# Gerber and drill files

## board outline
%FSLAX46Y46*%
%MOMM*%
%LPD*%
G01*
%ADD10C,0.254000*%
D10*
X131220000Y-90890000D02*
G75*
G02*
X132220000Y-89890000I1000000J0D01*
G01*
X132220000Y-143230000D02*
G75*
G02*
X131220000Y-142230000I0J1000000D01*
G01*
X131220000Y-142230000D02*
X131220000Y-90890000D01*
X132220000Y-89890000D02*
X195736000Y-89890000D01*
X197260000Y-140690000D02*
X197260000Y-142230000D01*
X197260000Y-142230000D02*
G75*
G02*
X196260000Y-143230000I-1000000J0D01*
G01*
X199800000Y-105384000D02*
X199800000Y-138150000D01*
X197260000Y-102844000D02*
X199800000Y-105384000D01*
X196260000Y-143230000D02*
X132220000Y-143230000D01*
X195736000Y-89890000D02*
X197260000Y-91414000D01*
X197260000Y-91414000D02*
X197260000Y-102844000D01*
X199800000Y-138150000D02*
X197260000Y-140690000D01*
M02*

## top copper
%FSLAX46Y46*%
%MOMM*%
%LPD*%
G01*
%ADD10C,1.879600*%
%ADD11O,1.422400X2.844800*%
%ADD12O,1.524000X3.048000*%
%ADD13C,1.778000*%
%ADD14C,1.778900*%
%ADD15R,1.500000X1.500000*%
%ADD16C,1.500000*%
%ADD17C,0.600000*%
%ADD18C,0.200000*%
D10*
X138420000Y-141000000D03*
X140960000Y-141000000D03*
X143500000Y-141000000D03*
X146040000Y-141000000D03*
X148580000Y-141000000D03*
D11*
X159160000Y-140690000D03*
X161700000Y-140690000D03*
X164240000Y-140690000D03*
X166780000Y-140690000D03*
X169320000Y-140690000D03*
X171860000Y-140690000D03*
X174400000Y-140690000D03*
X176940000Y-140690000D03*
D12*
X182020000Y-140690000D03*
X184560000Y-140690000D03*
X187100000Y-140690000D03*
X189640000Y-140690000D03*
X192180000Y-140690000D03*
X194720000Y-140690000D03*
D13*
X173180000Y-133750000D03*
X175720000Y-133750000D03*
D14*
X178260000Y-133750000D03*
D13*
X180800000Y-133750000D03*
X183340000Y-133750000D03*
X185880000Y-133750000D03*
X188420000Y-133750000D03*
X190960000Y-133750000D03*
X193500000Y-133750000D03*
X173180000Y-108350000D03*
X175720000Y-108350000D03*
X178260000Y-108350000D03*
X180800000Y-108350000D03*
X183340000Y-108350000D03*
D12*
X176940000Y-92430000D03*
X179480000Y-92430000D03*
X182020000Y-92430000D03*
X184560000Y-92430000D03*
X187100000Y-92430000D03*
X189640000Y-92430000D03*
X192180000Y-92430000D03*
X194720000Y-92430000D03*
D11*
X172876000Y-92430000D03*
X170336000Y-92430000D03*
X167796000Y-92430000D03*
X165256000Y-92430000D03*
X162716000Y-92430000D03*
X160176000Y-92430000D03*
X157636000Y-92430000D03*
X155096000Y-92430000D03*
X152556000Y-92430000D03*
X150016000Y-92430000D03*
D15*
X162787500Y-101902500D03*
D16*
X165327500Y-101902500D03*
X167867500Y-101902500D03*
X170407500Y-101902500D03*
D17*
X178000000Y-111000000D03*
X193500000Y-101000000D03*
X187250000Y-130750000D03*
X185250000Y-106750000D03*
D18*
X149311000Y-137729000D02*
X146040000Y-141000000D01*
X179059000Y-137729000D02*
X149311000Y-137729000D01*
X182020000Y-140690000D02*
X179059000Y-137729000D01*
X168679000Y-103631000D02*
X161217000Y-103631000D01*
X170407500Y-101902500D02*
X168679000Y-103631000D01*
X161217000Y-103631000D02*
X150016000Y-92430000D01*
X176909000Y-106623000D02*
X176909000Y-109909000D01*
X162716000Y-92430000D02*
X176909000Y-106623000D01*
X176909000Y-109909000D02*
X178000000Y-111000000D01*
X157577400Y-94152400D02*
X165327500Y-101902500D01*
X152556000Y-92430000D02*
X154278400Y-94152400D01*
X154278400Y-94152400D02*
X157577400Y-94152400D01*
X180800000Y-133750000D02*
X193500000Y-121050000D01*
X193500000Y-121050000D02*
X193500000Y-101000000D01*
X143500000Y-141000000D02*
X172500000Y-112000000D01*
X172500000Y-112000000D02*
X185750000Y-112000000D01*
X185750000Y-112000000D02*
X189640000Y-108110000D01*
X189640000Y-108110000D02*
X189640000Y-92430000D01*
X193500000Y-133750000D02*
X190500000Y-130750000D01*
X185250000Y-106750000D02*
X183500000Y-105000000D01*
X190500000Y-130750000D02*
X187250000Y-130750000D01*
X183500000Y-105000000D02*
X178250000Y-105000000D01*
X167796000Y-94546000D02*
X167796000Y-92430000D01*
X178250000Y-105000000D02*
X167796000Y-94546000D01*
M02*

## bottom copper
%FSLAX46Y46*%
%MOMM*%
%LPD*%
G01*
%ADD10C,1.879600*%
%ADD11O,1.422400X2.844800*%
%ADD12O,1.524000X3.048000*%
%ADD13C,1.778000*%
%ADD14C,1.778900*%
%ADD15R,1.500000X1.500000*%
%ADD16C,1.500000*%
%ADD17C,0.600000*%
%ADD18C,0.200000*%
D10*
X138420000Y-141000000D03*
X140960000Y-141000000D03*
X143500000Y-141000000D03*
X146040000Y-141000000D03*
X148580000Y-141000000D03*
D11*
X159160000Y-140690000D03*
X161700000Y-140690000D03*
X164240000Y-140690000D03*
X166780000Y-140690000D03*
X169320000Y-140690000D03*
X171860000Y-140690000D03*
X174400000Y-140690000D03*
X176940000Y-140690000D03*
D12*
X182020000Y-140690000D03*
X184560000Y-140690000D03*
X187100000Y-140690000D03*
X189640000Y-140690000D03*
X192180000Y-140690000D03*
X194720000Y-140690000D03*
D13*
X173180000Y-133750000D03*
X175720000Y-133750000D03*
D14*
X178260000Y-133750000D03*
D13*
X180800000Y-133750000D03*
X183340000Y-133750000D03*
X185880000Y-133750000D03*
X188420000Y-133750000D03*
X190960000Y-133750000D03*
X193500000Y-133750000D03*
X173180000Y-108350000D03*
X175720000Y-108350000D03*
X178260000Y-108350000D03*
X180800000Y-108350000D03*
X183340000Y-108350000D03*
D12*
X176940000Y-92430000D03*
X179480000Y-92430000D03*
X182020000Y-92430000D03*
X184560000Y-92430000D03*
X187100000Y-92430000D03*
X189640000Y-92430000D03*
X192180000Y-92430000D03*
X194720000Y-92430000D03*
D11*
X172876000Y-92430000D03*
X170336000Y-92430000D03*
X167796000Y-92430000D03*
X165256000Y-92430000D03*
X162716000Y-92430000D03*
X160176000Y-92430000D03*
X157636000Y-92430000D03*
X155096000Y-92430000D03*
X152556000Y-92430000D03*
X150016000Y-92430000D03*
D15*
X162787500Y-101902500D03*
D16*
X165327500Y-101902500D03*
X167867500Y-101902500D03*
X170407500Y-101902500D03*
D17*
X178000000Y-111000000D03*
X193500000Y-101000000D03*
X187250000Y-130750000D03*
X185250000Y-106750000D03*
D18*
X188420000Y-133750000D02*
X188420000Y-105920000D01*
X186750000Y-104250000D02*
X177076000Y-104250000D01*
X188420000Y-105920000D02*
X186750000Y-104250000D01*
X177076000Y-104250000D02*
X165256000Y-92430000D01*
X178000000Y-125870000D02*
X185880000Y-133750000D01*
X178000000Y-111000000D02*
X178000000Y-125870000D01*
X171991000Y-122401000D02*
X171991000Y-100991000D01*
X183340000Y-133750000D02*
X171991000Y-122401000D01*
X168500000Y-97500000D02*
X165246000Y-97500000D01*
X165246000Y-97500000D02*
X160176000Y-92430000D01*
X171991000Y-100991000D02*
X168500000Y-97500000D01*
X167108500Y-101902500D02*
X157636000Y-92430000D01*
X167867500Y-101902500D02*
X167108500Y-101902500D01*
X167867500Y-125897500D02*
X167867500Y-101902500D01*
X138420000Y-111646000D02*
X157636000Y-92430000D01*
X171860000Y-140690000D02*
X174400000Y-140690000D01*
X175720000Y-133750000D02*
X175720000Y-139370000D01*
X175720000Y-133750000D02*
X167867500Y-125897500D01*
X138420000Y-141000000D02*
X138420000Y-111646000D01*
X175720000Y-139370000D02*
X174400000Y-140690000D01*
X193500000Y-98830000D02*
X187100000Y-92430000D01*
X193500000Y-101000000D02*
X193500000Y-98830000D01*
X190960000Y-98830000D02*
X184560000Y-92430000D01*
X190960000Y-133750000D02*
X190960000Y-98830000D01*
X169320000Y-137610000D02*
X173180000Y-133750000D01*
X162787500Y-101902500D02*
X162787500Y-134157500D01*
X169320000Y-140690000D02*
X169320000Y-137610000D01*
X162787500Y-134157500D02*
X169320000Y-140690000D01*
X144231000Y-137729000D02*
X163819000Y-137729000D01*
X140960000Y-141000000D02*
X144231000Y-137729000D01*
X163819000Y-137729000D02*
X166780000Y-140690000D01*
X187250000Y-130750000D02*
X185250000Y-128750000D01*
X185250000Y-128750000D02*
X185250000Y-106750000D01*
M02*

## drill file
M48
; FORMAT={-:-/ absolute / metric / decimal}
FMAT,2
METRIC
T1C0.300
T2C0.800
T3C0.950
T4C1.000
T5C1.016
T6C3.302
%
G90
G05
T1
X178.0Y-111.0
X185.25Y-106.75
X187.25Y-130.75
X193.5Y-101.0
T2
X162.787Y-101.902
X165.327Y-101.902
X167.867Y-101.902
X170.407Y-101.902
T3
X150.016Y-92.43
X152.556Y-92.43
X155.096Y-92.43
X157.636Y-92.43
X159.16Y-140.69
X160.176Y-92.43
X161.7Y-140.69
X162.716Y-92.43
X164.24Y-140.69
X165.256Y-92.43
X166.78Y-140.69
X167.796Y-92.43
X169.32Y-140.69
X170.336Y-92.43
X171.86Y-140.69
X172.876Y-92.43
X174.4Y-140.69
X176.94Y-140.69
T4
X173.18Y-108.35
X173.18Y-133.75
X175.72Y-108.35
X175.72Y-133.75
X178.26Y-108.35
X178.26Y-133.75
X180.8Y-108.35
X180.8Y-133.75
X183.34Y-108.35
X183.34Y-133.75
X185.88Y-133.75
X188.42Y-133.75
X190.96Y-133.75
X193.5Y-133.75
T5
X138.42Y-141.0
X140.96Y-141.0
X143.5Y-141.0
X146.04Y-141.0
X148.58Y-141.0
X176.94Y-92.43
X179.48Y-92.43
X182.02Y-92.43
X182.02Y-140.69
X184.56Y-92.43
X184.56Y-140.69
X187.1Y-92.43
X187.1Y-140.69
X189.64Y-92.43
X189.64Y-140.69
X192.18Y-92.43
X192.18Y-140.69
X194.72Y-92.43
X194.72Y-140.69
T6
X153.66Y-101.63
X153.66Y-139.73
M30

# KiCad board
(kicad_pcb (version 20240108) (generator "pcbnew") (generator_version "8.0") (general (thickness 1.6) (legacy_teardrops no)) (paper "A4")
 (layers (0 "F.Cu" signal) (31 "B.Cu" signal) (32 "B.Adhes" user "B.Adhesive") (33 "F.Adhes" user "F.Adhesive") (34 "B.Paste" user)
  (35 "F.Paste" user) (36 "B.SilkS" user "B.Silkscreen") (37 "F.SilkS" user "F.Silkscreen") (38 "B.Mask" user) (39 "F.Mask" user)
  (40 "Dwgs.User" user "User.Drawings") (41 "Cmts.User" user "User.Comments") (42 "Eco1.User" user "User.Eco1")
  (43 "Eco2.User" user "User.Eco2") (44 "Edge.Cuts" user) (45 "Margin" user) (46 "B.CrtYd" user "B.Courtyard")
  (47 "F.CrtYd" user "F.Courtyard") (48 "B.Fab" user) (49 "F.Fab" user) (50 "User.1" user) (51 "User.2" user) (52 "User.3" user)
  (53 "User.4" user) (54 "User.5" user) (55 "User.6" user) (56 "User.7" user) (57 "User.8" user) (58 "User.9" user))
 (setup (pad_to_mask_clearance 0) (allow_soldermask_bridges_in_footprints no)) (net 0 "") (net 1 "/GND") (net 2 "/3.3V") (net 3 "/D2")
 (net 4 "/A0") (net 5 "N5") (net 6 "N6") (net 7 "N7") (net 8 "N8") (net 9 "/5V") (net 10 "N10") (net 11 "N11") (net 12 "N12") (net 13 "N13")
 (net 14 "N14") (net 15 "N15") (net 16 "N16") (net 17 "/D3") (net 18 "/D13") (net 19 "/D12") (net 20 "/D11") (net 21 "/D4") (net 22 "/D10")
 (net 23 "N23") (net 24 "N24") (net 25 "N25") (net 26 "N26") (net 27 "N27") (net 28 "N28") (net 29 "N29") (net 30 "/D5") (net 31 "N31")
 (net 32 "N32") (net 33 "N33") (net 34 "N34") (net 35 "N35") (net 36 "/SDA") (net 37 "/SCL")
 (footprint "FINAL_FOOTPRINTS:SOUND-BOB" (layer "F.Cu") (at 249.7736 -27.8211 -90)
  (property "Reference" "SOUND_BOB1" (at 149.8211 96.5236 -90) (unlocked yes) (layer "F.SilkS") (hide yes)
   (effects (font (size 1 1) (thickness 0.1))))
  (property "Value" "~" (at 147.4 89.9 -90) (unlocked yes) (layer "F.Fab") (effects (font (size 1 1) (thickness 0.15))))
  (pad "" np_thru_hole circle (at 129.4511 96.1136 270) (size 3.302 3.302) (drill 3.302) (layers "F&B.Cu" "*.Mask"))
  (pad "" np_thru_hole circle (at 167.5511 96.1136 270) (size 3.302 3.302) (drill 3.302) (layers "F&B.Cu" "*.Mask"))
  (pad "1" thru_hole circle (at 168.8211 111.3536 270) (size 1.8796 1.8796) (drill 1.016) (layers "*.Cu" "*.Mask") (remove_unused_layers no)
   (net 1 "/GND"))
  (pad "2" thru_hole circle (at 168.8211 108.8136 270) (size 1.8796 1.8796) (drill 1.016) (layers "*.Cu" "*.Mask") (remove_unused_layers no)
   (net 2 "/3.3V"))
  (pad "3" thru_hole circle (at 168.8211 106.2736 270) (size 1.8796 1.8796) (drill 1.016) (layers "*.Cu" "*.Mask") (remove_unused_layers no)
   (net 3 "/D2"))
  (pad "4" thru_hole circle (at 168.8211 103.7336 270) (size 1.8796 1.8796) (drill 1.016) (layers "*.Cu" "*.Mask") (remove_unused_layers no)
   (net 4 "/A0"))
  (pad "5" thru_hole circle (at 168.8211 101.1936 270) (size 1.8796 1.8796) (drill 1.016) (layers "*.Cu" "*.Mask") (remove_unused_layers no)
   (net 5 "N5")))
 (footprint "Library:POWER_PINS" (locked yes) (layer "F.Cu") (at 168.05 140.69)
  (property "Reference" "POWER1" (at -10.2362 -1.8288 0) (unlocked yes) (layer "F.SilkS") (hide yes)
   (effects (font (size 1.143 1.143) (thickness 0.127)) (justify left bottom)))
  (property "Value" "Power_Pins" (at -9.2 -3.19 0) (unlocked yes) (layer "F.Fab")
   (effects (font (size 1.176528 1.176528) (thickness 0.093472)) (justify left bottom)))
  (pad "1" thru_hole oval (at -8.89 0 90) (size 2.8448 1.4224) (drill 0.95) (layers "*.Cu" "*.Mask") (remove_unused_layers no) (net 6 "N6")
   (solder_mask_margin 0.0508) (thermal_bridge_angle 0))
  (pad "2" thru_hole oval (at -6.35 0 90) (size 2.8448 1.4224) (drill 0.95) (layers "*.Cu" "*.Mask") (remove_unused_layers no) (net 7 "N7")
   (solder_mask_margin 0.0508) (thermal_bridge_angle 0))
  (pad "3" thru_hole oval (at -3.81 0 90) (size 2.8448 1.4224) (drill 0.95) (layers "*.Cu" "*.Mask") (remove_unused_layers no) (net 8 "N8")
   (solder_mask_margin 0.0508) (thermal_bridge_angle 0))
  (pad "4" thru_hole oval (at -1.27 0 90) (size 2.8448 1.4224) (drill 0.95) (layers "*.Cu" "*.Mask") (remove_unused_layers no)
   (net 2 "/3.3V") (solder_mask_margin 0.0508) (thermal_bridge_angle 0))
  (pad "5" thru_hole oval (at 1.27 0 90) (size 2.8448 1.4224) (drill 0.95) (layers "*.Cu" "*.Mask") (remove_unused_layers no) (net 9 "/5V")
   (solder_mask_margin 0.0508) (thermal_bridge_angle 0))
  (pad "6" thru_hole oval (at 3.81 0 90) (size 2.8448 1.4224) (drill 0.95) (layers "*.Cu" "*.Mask") (remove_unused_layers no) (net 1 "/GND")
   (solder_mask_margin 0.0508) (thermal_bridge_angle 0))
  (pad "7" thru_hole oval (at 6.35 0 90) (size 2.8448 1.4224) (drill 0.95) (layers "*.Cu" "*.Mask") (remove_unused_layers no) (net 1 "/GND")
   (solder_mask_margin 0.0508) (thermal_bridge_angle 0))
  (pad "8" thru_hole oval (at 8.89 0 90) (size 2.8448 1.4224) (drill 0.95) (layers "*.Cu" "*.Mask") (remove_unused_layers no) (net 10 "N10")
   (solder_mask_margin 0.0508) (thermal_bridge_angle 0)))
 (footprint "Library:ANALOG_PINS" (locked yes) (layer "F.Cu") (at 188.37 140.69)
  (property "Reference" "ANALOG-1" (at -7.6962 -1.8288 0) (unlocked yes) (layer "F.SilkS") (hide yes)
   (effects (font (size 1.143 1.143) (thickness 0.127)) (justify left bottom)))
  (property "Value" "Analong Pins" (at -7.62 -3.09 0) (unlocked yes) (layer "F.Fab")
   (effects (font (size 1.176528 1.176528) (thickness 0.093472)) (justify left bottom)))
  (pad "1" thru_hole oval (at -6.35 0 90) (size 3.048 1.524) (drill 1.016) (layers "*.Cu" "*.Mask") (remove_unused_layers no) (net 4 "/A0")
   (solder_mask_margin 0.0508) (thermal_bridge_angle 0))
  (pad "2" thru_hole oval (at -3.81 0 90) (size 3.048 1.524) (drill 1.016) (layers "*.Cu" "*.Mask") (remove_unused_layers no) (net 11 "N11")
   (solder_mask_margin 0.0508) (thermal_bridge_angle 0))
  (pad "3" thru_hole oval (at -1.27 0 90) (size 3.048 1.524) (drill 1.016) (layers "*.Cu" "*.Mask") (remove_unused_layers no) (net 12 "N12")
   (solder_mask_margin 0.0508) (thermal_bridge_angle 0))
  (pad "4" thru_hole oval (at 1.27 0 90) (size 3.048 1.524) (drill 1.016) (layers "*.Cu" "*.Mask") (remove_unused_layers no) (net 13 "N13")
   (solder_mask_margin 0.0508) (thermal_bridge_angle 0))
  (pad "5" thru_hole oval (at 3.81 0 90) (size 3.048 1.524) (drill 1.016) (layers "*.Cu" "*.Mask") (remove_unused_layers no) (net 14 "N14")
   (solder_mask_margin 0.0508) (thermal_bridge_angle 0))
  (pad "6" thru_hole oval (at 6.35 0 90) (size 3.048 1.524) (drill 1.016) (layers "*.Cu" "*.Mask") (remove_unused_layers no) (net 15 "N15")
   (solder_mask_margin 0.0508) (thermal_bridge_angle 0)))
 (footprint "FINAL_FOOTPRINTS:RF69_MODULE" (layer "F.Cu") (at 35.0929 16.6814)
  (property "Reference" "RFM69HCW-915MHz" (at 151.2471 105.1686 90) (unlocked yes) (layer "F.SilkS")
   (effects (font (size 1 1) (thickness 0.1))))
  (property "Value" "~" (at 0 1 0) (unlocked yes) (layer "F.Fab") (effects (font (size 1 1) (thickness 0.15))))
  (pad "1" thru_hole circle (at 138.0871 117.0686 90) (size 1.778 1.778) (drill 1) (layers "*.Cu" "*.Mask") (remove_unused_layers no)
   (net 9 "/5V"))
  (pad "2" thru_hole circle (at 140.6271 117.0686 90) (size 1.778 1.778) (drill 1) (layers "*.Cu" "*.Mask") (remove_unused_layers no)
   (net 1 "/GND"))
  (pad "3" thru_hole circle (at 143.1671 117.0686) (size 1.7789 1.7789) (drill 1) (layers "*.Cu" "*.Mask") (remove_unused_layers no)
   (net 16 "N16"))
  (pad "4" thru_hole circle (at 145.7071 117.0686) (size 1.778 1.778) (drill 1) (layers "*.Cu" "*.Mask") (remove_unused_layers no)
   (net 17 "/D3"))
  (pad "5" thru_hole circle (at 148.2471 117.0686 90) (size 1.778 1.778) (drill 1) (layers "*.Cu" "*.Mask") (remove_unused_layers no)
   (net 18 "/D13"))
  (pad "6" thru_hole circle (at 150.7871 117.0686 90) (size 1.778 1.778) (drill 1) (layers "*.Cu" "*.Mask") (remove_unused_layers no)
   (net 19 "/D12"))
  (pad "7" thru_hole circle (at 153.3271 117.0686) (size 1.778 1.778) (drill 1) (layers "*.Cu" "*.Mask") (remove_unused_layers no)
   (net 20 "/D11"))
  (pad "8" thru_hole circle (at 155.8671 117.0686 90) (size 1.778 1.778) (drill 1) (layers "*.Cu" "*.Mask") (remove_unused_layers no)
   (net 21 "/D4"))
  (pad "9" thru_hole circle (at 158.4071 117.0686 90) (size 1.778 1.778) (drill 1) (layers "*.Cu" "*.Mask") (remove_unused_layers no)
   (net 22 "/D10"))
  (pad "10" thru_hole circle (at 138.0871 91.6686 90) (size 1.778 1.778) (drill 1) (layers "*.Cu" "*.Mask") (remove_unused_layers no)
   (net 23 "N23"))
  (pad "11" thru_hole circle (at 140.6271 91.6686 90) (size 1.778 1.778) (drill 1) (layers "*.Cu" "*.Mask") (remove_unused_layers no)
   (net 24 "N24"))
  (pad "12" thru_hole circle (at 143.1671 91.6686 90) (size 1.778 1.778) (drill 1) (layers "*.Cu" "*.Mask") (remove_unused_layers no)
   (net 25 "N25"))
  (pad "13" thru_hole circle (at 145.7071 91.6686 90) (size 1.778 1.778) (drill 1) (layers "*.Cu" "*.Mask") (remove_unused_layers no)
   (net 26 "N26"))
  (pad "14" thru_hole circle (at 148.2471 91.6686 90) (size 1.778 1.778) (drill 1) (layers "*.Cu" "*.Mask") (remove_unused_layers no)
   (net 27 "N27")))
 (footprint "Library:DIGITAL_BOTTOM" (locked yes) (layer "F.Cu") (at 185.83 92.43)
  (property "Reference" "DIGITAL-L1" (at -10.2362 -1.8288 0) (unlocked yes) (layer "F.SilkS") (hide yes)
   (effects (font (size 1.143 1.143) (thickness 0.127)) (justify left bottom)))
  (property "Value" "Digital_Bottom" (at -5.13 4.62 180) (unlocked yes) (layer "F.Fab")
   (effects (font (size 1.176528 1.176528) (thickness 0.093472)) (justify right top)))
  (pad "1" thru_hole oval (at -8.89 0 90) (size 3.048 1.524) (drill 1.016) (layers "*.Cu" "*.Mask") (remove_unused_layers no) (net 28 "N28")
   (solder_mask_margin 0.0508) (thermal_bridge_angle 0))
  (pad "2" thru_hole oval (at -6.35 0 90) (size 3.048 1.524) (drill 1.016) (layers "*.Cu" "*.Mask") (remove_unused_layers no) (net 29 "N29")
   (solder_mask_margin 0.0508) (thermal_bridge_angle 0))
  (pad "3" thru_hole oval (at -3.81 0 90) (size 3.048 1.524) (drill 1.016) (layers "*.Cu" "*.Mask") (remove_unused_layers no) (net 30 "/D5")
   (solder_mask_margin 0.0508) (thermal_bridge_angle 0))
  (pad "4" thru_hole oval (at -1.27 0 90) (size 3.048 1.524) (drill 1.016) (layers "*.Cu" "*.Mask") (remove_unused_layers no) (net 21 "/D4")
   (solder_mask_margin 0.0508) (thermal_bridge_angle 0))
  (pad "5" thru_hole oval (at 1.27 0 90) (size 3.048 1.524) (drill 1.016) (layers "*.Cu" "*.Mask") (remove_unused_layers no) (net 17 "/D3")
   (solder_mask_margin 0.0508) (thermal_bridge_angle 0))
  (pad "6" thru_hole oval (at 3.81 0 90) (size 3.048 1.524) (drill 1.016) (layers "*.Cu" "*.Mask") (remove_unused_layers no) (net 3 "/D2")
   (solder_mask_margin 0.0508) (thermal_bridge_angle 0))
  (pad "7" thru_hole oval (at 6.35 0 90) (size 3.048 1.524) (drill 1.016) (layers "*.Cu" "*.Mask") (remove_unused_layers no) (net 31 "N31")
   (solder_mask_margin 0.0508) (thermal_bridge_angle 0))
  (pad "8" thru_hole oval (at 8.89 0 90) (size 3.048 1.524) (drill 1.016) (layers "*.Cu" "*.Mask") (remove_unused_layers no) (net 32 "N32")
   (solder_mask_margin 0.0508) (thermal_bridge_angle 0)))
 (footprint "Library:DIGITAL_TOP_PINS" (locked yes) (layer "F.Cu") (at 161.446 92.43 180)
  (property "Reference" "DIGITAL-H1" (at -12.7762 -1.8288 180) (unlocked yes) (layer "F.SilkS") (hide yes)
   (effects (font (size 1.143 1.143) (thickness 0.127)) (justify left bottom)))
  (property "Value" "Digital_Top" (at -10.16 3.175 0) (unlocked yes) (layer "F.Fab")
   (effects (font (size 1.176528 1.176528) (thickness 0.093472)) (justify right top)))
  (pad "1" thru_hole oval (at -11.43 0 270) (size 2.8448 1.4224) (drill 0.95) (layers "*.Cu" "*.Mask") (remove_unused_layers no)
   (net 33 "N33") (solder_mask_margin 0.0508) (thermal_bridge_angle 0))
  (pad "2" thru_hole oval (at -8.89 0 270) (size 2.8448 1.4224) (drill 0.95) (layers "*.Cu" "*.Mask") (remove_unused_layers no)
   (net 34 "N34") (solder_mask_margin 0.0508) (thermal_bridge_angle 0))
  (pad "3" thru_hole oval (at -6.35 0 270) (size 2.8448 1.4224) (drill 0.95) (layers "*.Cu" "*.Mask") (remove_unused_layers no)
   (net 22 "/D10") (solder_mask_margin 0.0508) (thermal_bridge_angle 0))
  (pad "4" thru_hole oval (at -3.81 0 270) (size 2.8448 1.4224) (drill 0.95) (layers "*.Cu" "*.Mask") (remove_unused_layers no)
   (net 20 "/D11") (solder_mask_margin 0.0508) (thermal_bridge_angle 0))
  (pad "5" thru_hole oval (at -1.27 0 270) (size 2.8448 1.4224) (drill 0.95) (layers "*.Cu" "*.Mask") (remove_unused_layers no)
   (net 19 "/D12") (solder_mask_margin 0.0508) (thermal_bridge_angle 0))
  (pad "6" thru_hole oval (at 1.27 0 270) (size 2.8448 1.4224) (drill 0.95) (layers "*.Cu" "*.Mask") (remove_unused_layers no)
   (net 18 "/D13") (solder_mask_margin 0.0508) (thermal_bridge_angle 0))
  (pad "7" thru_hole oval (at 3.81 0 270) (size 2.8448 1.4224) (drill 0.95) (layers "*.Cu" "*.Mask") (remove_unused_layers no)
   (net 1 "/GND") (solder_mask_margin 0.0508) (thermal_bridge_angle 0))
  (pad "8" thru_hole oval (at 6.35 0 270) (size 2.8448 1.4224) (drill 0.95) (layers "*.Cu" "*.Mask") (remove_unused_layers no)
   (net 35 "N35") (solder_mask_margin 0.0508) (thermal_bridge_angle 0))
  (pad "9" thru_hole oval (at 8.89 0 270) (size 2.8448 1.4224) (drill 0.95) (layers "*.Cu" "*.Mask") (remove_unused_layers no)
   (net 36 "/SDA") (solder_mask_margin 0.0508) (thermal_bridge_angle 0))
  (pad "10" thru_hole oval (at 11.43 0 270) (size 2.8448 1.4224) (drill 0.95) (layers "*.Cu" "*.Mask") (remove_unused_layers no)
   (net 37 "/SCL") (solder_mask_margin 0.0508) (thermal_bridge_angle 0)))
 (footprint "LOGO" (layer "F.Cu") (at 138.25 94.25)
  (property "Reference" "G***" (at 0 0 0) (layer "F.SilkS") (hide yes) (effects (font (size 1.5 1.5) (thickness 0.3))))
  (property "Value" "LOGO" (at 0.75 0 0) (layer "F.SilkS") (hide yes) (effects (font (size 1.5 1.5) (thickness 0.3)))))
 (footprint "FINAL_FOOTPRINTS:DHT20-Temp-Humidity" (layer "F.Cu") (at 162.7875 101.9025 90)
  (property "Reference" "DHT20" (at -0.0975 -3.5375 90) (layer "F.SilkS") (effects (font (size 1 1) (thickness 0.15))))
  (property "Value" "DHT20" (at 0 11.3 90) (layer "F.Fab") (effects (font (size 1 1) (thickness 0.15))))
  (pad "1" thru_hole rect (at 0 0 90) (size 1.5 1.5) (drill 0.8) (layers "*.Cu" "*.Mask") (remove_unused_layers no) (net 9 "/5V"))
  (pad "2" thru_hole circle (at 0 2.54 90) (size 1.5 1.5) (drill 0.8) (layers "*.Cu" "*.Mask") (remove_unused_layers no) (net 36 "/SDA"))
  (pad "3" thru_hole circle (at 0 5.08 90) (size 1.5 1.5) (drill 0.8) (layers "*.Cu" "*.Mask") (remove_unused_layers no) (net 1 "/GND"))
  (pad "4" thru_hole circle (at 0 7.62 90) (size 1.5 1.5) (drill 0.8) (layers "*.Cu" "*.Mask") (remove_unused_layers no) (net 37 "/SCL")))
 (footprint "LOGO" (layer "B.Cu") (at 153 130.25 180)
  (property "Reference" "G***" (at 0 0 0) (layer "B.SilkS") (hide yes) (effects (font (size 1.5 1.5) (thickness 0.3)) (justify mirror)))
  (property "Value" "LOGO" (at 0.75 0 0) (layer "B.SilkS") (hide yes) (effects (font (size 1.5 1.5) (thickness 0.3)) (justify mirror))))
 (gr_arc (start 131.22 90.89) (mid 131.512893 90.182893) (end 132.22 89.89) (stroke (width 0.254) (type solid)) (layer "Edge.Cuts"))
 (gr_arc (start 132.22 143.23) (mid 131.512893 142.937107) (end 131.22 142.23) (stroke (width 0.254) (type solid)) (layer "Edge.Cuts"))
 (gr_line (start 131.22 142.23) (end 131.22 90.89) (stroke (width 0.254) (type solid)) (layer "Edge.Cuts"))
 (gr_line (start 132.22 89.89) (end 195.736 89.89) (stroke (width 0.254) (type solid)) (layer "Edge.Cuts"))
 (gr_line (start 197.26 140.69) (end 197.26 142.23) (stroke (width 0.254) (type solid)) (layer "Edge.Cuts"))
 (gr_arc (start 197.26 142.23) (mid 196.967107 142.937107) (end 196.26 143.23) (stroke (width 0.254) (type solid)) (layer "Edge.Cuts"))
 (gr_line (start 199.8 105.384) (end 199.8 138.15) (stroke (width 0.254) (type solid)) (layer "Edge.Cuts"))
 (gr_line (start 197.26 102.844) (end 199.8 105.384) (stroke (width 0.254) (type solid)) (layer "Edge.Cuts"))
 (gr_line (start 196.26 143.23) (end 132.22 143.23) (stroke (width 0.254) (type solid)) (layer "Edge.Cuts"))
 (gr_line (start 195.736 89.89) (end 197.26 91.414) (stroke (width 0.254) (type solid)) (layer "Edge.Cuts"))
 (gr_line (start 197.26 91.414) (end 197.26 102.844) (stroke (width 0.254) (type solid)) (layer "Edge.Cuts"))
 (gr_line (start 199.8 138.15) (end 197.26 140.69) (stroke (width 0.254) (type solid)) (layer "Edge.Cuts"))
 (segment (start 149.311 137.729) (end 146.04 141) (width 0.2) (layer "F.Cu") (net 4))
 (segment (start 179.059 137.729) (end 149.311 137.729) (width 0.2) (layer "F.Cu") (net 4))
 (segment (start 182.02 140.69) (end 179.059 137.729) (width 0.2) (layer "F.Cu") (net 4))
 (segment (start 188.42 133.75) (end 188.42 105.92) (width 0.2) (layer "B.Cu") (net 20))
 (segment (start 186.75 104.25) (end 177.076 104.25) (width 0.2) (layer "B.Cu") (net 20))
 (segment (start 188.42 105.92) (end 186.75 104.25) (width 0.2) (layer "B.Cu") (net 20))
 (segment (start 177.076 104.25) (end 165.256 92.43) (width 0.2) (layer "B.Cu") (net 20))
 (segment (start 168.679 103.631) (end 161.217 103.631) (width 0.2) (layer "F.Cu") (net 37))
 (segment (start 170.4075 101.9025) (end 168.679 103.631) (width 0.2) (layer "F.Cu") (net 37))
 (segment (start 161.217 103.631) (end 150.016 92.43) (width 0.2) (layer "F.Cu") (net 37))
 (segment (start 176.909 106.623) (end 176.909 109.909) (width 0.2) (layer "F.Cu") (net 19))
 (segment (start 162.716 92.43) (end 176.909 106.623) (width 0.2) (layer "F.Cu") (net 19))
 (segment (start 176.909 109.909) (end 178 111) (width 0.2) (layer "F.Cu") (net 19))
 (via (at 178 111) (size 0.6) (drill 0.3) (layers "F.Cu" "B.Cu") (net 19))
 (segment (start 178 125.87) (end 185.88 133.75) (width 0.2) (layer "B.Cu") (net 19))
 (segment (start 178 111) (end 178 125.87) (width 0.2) (layer "B.Cu") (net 19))
 (segment (start 171.991 122.401) (end 171.991 100.991) (width 0.2) (layer "B.Cu") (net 18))
 (segment (start 183.34 133.75) (end 171.991 122.401) (width 0.2) (layer "B.Cu") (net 18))
 (segment (start 168.5 97.5) (end 165.246 97.5) (width 0.2) (layer "B.Cu") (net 18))
 (segment (start 165.246 97.5) (end 160.176 92.43) (width 0.2) (layer "B.Cu") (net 18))
 (segment (start 171.991 100.991) (end 168.5 97.5) (width 0.2) (layer "B.Cu") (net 18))
 (segment (start 157.5774 94.1524) (end 165.3275 101.9025) (width 0.2) (layer "F.Cu") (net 36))
 (segment (start 152.556 92.43) (end 154.2784 94.1524) (width 0.2) (layer "F.Cu") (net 36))
 (segment (start 154.2784 94.1524) (end 157.5774 94.1524) (width 0.2) (layer "F.Cu") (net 36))
 (segment (start 167.1085 101.9025) (end 157.636 92.43) (width 0.2) (layer "B.Cu") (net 1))
 (segment (start 167.8675 101.9025) (end 167.1085 101.9025) (width 0.2) (layer "B.Cu") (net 1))
 (segment (start 167.8675 125.8975) (end 167.8675 101.9025) (width 0.2) (layer "B.Cu") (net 1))
 (segment (start 138.42 111.646) (end 157.636 92.43) (width 0.2) (layer "B.Cu") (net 1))
 (segment (start 171.86 140.69) (end 174.4 140.69) (width 0.2) (layer "B.Cu") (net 1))
 (segment (start 175.72 133.75) (end 175.72 139.37) (width 0.2) (layer "B.Cu") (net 1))
 (segment (start 175.72 133.75) (end 167.8675 125.8975) (width 0.2) (layer "B.Cu") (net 1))
 (segment (start 138.42 141) (end 138.42 111.646) (width 0.2) (layer "B.Cu") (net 1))
 (segment (start 175.72 139.37) (end 174.4 140.69) (width 0.2) (layer "B.Cu") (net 1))
 (segment (start 180.8 133.75) (end 193.5 121.05) (width 0.2) (layer "F.Cu") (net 17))
 (segment (start 193.5 121.05) (end 193.5 101) (width 0.2) (layer "F.Cu") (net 17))
 (via (at 193.5 101) (size 0.6) (drill 0.3) (layers "F.Cu" "B.Cu") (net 17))
 (segment (start 193.5 98.83) (end 187.1 92.43) (width 0.2) (layer "B.Cu") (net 17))
 (segment (start 193.5 101) (end 193.5 98.83) (width 0.2) (layer "B.Cu") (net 17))
 (segment (start 190.96 98.83) (end 184.56 92.43) (width 0.2) (layer "B.Cu") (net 21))
 (segment (start 190.96 133.75) (end 190.96 98.83) (width 0.2) (layer "B.Cu") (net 21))
 (segment (start 143.5 141) (end 172.5 112) (width 0.2) (layer "F.Cu") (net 3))
 (segment (start 172.5 112) (end 185.75 112) (width 0.2) (layer "F.Cu") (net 3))
 (segment (start 185.75 112) (end 189.64 108.11) (width 0.2) (layer "F.Cu") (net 3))
 (segment (start 189.64 108.11) (end 189.64 92.43) (width 0.2) (layer "F.Cu") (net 3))
 (segment (start 169.32 137.61) (end 173.18 133.75) (width 0.2) (layer "B.Cu") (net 9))
 (segment (start 162.7875 101.9025) (end 162.7875 134.1575) (width 0.2) (layer "B.Cu") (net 9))
 (segment (start 169.32 140.69) (end 169.32 137.61) (width 0.2) (layer "B.Cu") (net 9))
 (segment (start 162.7875 134.1575) (end 169.32 140.69) (width 0.2) (layer "B.Cu") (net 9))
 (segment (start 144.231 137.729) (end 163.819 137.729) (width 0.2) (layer "B.Cu") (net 2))
 (segment (start 140.96 141) (end 144.231 137.729) (width 0.2) (layer "B.Cu") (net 2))
 (segment (start 163.819 137.729) (end 166.78 140.69) (width 0.2) (layer "B.Cu") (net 2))
 (segment (start 193.5 133.75) (end 190.5 130.75) (width 0.2) (layer "F.Cu") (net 22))
 (segment (start 185.25 106.75) (end 183.5 105) (width 0.2) (layer "F.Cu") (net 22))
 (segment (start 190.5 130.75) (end 187.25 130.75) (width 0.2) (layer "F.Cu") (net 22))
 (segment (start 183.5 105) (end 178.25 105) (width 0.2) (layer "F.Cu") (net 22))
 (segment (start 167.796 94.546) (end 167.796 92.43) (width 0.2) (layer "F.Cu") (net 22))
 (segment (start 178.25 105) (end 167.796 94.546) (width 0.2) (layer "F.Cu") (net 22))
 (via (at 187.25 130.75) (size 0.6) (drill 0.3) (layers "F.Cu" "B.Cu") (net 22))
 (via (at 185.25 106.75) (size 0.6) (drill 0.3) (layers "F.Cu" "B.Cu") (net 22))
 (segment (start 187.25 130.75) (end 185.25 128.75) (width 0.2) (layer "B.Cu") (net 22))
 (segment (start 185.25 128.75) (end 185.25 106.75) (width 0.2) (layer "B.Cu") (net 22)))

